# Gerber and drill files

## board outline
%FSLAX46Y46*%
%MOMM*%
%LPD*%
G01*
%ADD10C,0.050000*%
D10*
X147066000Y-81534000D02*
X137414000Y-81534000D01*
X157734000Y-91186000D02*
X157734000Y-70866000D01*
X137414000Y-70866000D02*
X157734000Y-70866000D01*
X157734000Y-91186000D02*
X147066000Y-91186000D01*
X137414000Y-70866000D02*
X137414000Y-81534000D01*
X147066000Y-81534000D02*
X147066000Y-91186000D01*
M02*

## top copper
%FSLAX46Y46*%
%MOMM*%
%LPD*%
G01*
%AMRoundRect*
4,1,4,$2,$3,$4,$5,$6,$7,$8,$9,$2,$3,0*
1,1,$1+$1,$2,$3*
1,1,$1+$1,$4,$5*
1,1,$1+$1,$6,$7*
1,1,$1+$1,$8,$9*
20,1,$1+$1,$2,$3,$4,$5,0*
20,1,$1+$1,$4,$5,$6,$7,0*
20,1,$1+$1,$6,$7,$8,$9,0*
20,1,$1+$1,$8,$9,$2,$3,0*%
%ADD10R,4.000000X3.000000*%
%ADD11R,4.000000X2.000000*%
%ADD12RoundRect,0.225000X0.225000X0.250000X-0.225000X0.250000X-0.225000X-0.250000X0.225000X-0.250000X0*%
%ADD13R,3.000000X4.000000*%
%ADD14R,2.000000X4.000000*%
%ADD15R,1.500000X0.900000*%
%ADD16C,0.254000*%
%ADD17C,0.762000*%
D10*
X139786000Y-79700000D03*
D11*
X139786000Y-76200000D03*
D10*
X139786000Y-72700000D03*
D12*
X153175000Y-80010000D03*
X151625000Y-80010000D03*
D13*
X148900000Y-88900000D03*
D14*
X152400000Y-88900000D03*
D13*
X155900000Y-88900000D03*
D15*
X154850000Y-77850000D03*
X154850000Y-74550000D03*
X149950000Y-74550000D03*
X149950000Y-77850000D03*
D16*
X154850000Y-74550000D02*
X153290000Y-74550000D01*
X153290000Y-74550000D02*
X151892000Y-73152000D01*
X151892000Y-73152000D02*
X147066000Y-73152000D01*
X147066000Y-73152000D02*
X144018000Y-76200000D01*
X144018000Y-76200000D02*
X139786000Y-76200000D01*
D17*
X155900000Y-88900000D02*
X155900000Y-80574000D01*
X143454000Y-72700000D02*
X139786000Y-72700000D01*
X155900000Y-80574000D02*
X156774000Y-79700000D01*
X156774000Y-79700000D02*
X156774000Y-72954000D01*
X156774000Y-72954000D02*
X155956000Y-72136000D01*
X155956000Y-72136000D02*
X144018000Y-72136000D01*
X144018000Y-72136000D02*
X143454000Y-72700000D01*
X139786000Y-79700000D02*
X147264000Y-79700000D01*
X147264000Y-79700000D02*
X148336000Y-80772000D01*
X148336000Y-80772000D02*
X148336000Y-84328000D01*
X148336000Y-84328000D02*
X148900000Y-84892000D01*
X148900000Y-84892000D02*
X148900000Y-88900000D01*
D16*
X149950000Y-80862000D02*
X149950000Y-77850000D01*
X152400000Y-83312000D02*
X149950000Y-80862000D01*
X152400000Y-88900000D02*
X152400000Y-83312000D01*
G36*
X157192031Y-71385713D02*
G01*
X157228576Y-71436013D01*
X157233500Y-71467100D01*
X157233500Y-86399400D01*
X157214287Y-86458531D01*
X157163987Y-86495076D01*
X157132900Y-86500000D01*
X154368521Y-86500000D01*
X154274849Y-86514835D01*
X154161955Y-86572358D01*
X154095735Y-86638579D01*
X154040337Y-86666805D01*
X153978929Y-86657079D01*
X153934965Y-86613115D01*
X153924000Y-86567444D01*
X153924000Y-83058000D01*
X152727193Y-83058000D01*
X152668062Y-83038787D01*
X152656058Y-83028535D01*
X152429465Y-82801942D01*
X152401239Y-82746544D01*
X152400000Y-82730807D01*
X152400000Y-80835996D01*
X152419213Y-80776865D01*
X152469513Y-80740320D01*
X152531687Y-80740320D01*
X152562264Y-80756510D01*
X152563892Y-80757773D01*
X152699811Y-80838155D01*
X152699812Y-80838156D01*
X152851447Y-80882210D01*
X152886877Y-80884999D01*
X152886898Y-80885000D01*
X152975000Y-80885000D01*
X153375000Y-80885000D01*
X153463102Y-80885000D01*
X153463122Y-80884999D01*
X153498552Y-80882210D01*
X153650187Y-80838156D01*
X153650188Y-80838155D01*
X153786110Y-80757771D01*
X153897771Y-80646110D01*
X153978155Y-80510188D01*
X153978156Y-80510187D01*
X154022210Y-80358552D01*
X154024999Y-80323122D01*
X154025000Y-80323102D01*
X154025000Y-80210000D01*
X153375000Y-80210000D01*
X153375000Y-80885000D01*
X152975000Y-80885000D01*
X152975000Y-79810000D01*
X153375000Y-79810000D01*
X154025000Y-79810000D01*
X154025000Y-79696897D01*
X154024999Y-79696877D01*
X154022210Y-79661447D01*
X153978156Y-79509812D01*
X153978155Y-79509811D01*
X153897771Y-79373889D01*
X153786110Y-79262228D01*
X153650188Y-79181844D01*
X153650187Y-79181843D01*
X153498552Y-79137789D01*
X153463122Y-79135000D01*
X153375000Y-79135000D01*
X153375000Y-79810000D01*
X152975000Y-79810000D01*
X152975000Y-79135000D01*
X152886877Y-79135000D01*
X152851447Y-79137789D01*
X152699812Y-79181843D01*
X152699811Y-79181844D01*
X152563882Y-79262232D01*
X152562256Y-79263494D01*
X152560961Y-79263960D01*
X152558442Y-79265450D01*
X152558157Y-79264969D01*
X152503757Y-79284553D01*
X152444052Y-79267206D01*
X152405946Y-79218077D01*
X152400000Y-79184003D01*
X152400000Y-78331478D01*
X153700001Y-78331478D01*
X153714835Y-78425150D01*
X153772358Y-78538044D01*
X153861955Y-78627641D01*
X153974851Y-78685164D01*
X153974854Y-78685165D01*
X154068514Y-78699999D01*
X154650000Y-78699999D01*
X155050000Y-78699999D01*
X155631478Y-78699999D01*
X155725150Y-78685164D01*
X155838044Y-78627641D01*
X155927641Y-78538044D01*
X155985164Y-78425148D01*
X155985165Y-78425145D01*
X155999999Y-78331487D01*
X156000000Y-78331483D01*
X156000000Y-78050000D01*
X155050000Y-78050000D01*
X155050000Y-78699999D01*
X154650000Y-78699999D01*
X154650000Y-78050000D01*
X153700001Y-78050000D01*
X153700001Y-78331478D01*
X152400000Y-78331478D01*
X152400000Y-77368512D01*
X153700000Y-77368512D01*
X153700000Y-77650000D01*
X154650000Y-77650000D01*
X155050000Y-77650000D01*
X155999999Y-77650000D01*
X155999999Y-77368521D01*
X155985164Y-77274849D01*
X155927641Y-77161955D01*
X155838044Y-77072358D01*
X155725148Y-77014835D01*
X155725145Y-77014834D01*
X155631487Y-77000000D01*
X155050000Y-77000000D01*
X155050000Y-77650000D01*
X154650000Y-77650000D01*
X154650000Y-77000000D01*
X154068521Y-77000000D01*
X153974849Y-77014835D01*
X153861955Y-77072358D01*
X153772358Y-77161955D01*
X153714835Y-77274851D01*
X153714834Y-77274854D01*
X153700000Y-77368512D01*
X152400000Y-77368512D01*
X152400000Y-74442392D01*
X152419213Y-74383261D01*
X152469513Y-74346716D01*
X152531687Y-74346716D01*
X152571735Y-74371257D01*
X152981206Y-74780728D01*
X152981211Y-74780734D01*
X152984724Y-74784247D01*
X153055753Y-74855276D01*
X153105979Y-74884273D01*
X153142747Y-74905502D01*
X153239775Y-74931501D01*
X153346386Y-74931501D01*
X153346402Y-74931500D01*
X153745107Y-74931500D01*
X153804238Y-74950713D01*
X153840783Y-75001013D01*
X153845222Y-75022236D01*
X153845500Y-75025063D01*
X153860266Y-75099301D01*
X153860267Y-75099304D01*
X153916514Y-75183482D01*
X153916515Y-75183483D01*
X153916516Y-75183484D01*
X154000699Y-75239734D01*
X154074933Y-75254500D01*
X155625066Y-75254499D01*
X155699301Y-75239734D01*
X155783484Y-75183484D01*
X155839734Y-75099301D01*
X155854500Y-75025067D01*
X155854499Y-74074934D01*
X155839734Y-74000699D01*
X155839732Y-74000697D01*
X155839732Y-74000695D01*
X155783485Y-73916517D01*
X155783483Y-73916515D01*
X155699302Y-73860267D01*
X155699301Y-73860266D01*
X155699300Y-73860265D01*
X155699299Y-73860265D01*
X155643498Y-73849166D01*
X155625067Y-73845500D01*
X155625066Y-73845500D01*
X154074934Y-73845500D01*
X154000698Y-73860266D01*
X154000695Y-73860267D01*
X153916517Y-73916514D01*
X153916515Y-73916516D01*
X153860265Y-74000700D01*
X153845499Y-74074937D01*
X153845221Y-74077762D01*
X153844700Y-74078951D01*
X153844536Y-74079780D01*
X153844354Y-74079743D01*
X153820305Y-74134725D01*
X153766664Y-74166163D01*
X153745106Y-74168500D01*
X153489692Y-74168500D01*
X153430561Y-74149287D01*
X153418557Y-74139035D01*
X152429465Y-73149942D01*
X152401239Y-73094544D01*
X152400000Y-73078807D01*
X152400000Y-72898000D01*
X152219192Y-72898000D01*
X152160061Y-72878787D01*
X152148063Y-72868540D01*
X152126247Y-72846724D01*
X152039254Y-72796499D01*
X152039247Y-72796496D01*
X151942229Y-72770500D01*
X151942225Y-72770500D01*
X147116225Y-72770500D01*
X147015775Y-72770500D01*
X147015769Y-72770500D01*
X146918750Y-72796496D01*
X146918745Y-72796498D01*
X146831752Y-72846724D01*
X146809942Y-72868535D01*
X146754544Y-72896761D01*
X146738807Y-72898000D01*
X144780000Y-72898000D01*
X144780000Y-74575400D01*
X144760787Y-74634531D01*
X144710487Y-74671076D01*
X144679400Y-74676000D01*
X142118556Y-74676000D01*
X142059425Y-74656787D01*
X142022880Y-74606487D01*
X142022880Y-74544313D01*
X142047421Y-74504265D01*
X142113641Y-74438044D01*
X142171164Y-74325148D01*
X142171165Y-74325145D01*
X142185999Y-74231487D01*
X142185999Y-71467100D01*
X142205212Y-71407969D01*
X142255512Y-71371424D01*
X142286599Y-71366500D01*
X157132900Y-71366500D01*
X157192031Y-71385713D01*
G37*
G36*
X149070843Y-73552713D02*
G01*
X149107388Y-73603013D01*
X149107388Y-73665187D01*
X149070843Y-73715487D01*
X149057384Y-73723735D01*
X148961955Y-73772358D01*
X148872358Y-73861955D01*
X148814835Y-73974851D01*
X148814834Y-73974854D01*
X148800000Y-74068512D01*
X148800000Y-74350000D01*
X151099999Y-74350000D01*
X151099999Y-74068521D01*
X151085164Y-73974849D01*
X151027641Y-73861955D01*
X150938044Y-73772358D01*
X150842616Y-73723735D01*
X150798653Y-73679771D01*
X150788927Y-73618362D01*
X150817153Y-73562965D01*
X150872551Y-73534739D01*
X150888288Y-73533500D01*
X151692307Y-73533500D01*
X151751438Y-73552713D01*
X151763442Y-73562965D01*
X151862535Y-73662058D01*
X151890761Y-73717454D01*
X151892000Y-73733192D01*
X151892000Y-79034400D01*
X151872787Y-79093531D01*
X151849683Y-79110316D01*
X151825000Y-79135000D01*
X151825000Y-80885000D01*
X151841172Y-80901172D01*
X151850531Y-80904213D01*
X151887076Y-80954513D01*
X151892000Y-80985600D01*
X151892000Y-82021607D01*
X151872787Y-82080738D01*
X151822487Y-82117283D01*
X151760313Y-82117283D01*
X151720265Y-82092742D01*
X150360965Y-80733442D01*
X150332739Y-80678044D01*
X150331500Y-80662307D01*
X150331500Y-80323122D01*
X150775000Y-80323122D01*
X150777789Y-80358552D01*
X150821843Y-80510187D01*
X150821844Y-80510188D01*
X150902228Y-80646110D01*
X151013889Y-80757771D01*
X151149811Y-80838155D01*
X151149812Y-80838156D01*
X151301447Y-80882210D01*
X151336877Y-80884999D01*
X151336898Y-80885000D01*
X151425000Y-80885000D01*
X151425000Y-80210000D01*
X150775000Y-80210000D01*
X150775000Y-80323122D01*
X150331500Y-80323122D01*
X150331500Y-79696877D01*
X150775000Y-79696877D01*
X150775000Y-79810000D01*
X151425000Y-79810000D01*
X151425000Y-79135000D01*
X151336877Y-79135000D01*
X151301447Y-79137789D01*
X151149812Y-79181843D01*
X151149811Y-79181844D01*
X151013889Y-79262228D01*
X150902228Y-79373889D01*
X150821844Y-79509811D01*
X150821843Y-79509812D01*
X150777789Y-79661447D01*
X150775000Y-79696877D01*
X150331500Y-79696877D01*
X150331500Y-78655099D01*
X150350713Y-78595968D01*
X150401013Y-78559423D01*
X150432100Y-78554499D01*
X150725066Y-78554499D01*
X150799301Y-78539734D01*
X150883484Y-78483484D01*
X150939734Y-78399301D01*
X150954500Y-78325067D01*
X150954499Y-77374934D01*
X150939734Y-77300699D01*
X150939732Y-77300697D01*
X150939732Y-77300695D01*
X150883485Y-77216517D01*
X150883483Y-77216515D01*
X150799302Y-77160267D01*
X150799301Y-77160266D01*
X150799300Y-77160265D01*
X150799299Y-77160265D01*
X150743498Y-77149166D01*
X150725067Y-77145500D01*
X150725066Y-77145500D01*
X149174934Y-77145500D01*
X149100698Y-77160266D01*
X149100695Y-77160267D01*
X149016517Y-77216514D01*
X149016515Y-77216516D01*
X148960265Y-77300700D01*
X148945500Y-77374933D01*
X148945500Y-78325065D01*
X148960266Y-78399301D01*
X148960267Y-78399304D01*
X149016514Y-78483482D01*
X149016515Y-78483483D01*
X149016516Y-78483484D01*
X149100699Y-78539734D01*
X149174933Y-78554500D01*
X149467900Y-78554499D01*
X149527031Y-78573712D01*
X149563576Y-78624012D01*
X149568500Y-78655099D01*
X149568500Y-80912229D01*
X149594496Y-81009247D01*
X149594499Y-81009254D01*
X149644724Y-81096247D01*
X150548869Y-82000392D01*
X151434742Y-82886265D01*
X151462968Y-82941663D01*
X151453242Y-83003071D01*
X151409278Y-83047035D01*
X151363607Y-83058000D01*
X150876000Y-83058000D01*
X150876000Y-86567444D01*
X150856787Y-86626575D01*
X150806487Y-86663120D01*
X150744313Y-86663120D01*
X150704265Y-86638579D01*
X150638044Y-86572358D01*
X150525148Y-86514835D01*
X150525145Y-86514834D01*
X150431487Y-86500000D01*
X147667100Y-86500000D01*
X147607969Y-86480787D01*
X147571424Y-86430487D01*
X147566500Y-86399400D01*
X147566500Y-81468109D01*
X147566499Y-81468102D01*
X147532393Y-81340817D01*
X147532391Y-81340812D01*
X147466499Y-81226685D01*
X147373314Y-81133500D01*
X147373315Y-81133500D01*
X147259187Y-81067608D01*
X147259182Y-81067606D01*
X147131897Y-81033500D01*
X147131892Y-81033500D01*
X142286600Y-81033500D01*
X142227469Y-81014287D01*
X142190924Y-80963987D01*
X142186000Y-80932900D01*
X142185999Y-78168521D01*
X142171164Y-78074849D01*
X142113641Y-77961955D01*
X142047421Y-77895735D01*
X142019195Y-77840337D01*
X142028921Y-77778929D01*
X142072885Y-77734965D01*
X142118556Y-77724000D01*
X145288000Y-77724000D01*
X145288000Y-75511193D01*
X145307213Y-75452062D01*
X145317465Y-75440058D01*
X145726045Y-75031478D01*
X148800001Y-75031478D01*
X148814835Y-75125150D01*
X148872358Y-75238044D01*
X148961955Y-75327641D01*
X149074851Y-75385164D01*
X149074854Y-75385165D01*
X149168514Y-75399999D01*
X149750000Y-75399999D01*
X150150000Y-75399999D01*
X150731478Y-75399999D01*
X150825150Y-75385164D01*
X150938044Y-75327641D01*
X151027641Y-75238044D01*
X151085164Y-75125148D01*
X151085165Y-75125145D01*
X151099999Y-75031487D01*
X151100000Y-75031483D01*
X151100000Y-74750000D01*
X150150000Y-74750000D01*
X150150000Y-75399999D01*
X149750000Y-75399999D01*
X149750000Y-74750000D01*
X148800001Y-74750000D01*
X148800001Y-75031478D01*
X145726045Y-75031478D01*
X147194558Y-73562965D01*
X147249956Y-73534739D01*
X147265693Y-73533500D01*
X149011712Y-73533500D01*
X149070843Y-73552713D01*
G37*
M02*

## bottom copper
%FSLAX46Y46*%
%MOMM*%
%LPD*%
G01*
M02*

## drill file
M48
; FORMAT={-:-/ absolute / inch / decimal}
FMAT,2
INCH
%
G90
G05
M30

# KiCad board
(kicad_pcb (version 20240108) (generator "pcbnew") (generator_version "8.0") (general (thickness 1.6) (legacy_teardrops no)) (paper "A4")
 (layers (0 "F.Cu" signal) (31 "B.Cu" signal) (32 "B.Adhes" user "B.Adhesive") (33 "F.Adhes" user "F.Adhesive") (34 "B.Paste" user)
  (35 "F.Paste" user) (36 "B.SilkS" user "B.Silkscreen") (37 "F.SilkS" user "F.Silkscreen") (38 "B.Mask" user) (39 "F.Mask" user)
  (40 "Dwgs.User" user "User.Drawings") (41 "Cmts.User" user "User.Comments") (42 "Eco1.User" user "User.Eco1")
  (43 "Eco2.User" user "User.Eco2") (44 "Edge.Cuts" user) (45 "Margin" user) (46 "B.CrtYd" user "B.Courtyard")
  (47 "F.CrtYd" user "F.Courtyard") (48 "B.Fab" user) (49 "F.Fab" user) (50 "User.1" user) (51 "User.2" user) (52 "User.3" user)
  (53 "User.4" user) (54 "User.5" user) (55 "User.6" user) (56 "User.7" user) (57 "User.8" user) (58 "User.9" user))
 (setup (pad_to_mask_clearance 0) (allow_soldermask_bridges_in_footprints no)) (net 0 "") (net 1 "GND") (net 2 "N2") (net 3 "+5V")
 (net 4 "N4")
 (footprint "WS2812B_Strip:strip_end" (layer "F.Cu") (at 139.786 76.2 180)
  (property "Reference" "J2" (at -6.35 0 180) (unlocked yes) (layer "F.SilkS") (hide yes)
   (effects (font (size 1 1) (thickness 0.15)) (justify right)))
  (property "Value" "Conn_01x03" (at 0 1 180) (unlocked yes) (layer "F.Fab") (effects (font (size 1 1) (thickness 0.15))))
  (pad "1" smd rect (at 0 -3.5 180) (size 4 3) (layers "F.Cu" "F.Paste" "F.Mask") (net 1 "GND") (thermal_bridge_angle 45))
  (pad "2" smd rect (at 0 0 180) (size 4 2) (layers "F.Cu" "F.Paste" "F.Mask") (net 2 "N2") (thermal_bridge_angle 45))
  (pad "3" smd rect (at 0 3.5 180) (size 4 3) (layers "F.Cu" "F.Paste" "F.Mask") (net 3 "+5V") (thermal_bridge_angle 45)))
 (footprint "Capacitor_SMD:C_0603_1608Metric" (layer "F.Cu") (at 152.4 80.01 180)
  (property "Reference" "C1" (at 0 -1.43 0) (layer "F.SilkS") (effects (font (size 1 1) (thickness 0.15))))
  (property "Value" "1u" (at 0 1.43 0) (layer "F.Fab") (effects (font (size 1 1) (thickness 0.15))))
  (pad "1" smd roundrect (at -0.775 0 180) (size 0.9 0.95) (layers "F.Cu" "F.Paste" "F.Mask") (roundrect_rratio 0.25) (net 3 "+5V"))
  (pad "2" smd roundrect (at 0.775 0 180) (size 0.9 0.95) (layers "F.Cu" "F.Paste" "F.Mask") (roundrect_rratio 0.25) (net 1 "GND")))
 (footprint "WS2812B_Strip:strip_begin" (layer "F.Cu") (at 152.4 88.9 90)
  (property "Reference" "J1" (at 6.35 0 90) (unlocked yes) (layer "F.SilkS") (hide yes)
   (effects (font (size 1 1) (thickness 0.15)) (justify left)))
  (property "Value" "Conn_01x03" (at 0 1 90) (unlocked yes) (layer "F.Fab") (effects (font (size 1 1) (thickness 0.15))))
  (pad "1" smd rect (at 0 -3.5 90) (size 4 3) (layers "F.Cu" "F.Paste" "F.Mask") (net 1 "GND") (thermal_bridge_angle 45))
  (pad "2" smd rect (at 0 0 90) (size 4 2) (layers "F.Cu" "F.Paste" "F.Mask") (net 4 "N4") (thermal_bridge_angle 45))
  (pad "3" smd rect (at 0 3.5 90) (size 4 3) (layers "F.Cu" "F.Paste" "F.Mask") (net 3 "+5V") (thermal_bridge_angle 45)))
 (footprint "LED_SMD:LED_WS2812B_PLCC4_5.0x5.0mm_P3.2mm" (layer "F.Cu") (at 152.4 76.2 180)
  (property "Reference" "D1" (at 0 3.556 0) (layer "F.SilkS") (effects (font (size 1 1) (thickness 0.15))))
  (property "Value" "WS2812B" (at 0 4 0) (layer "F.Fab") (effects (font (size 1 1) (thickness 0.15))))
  (pad "1" smd rect (at -2.45 -1.65 180) (size 1.5 0.9) (layers "F.Cu" "F.Paste" "F.Mask") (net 3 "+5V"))
  (pad "2" smd rect (at -2.45 1.65 180) (size 1.5 0.9) (layers "F.Cu" "F.Paste" "F.Mask") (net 2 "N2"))
  (pad "3" smd rect (at 2.45 1.65 180) (size 1.5 0.9) (layers "F.Cu" "F.Paste" "F.Mask") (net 1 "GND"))
  (pad "4" smd rect (at 2.45 -1.65 180) (size 1.5 0.9) (layers "F.Cu" "F.Paste" "F.Mask") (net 4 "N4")))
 (gr_line (start 147.066 81.534) (end 137.414 81.534) (stroke (width 0.05) (type default)) (layer "Edge.Cuts"))
 (gr_line (start 157.734 91.186) (end 157.734 70.866) (stroke (width 0.05) (type default)) (layer "Edge.Cuts"))
 (gr_line (start 137.414 70.866) (end 157.734 70.866) (stroke (width 0.05) (type default)) (layer "Edge.Cuts"))
 (gr_line (start 157.734 91.186) (end 147.066 91.186) (stroke (width 0.05) (type default)) (layer "Edge.Cuts"))
 (gr_line (start 137.414 70.866) (end 137.414 81.534) (stroke (width 0.05) (type default)) (layer "Edge.Cuts"))
 (gr_line (start 147.066 81.534) (end 147.066 91.186) (stroke (width 0.05) (type default)) (layer "Edge.Cuts"))
 (segment (start 149.95 80.862) (end 149.95 77.85) (width 0.254) (layer "F.Cu") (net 4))
 (segment (start 152.4 83.312) (end 149.95 80.862) (width 0.254) (layer "F.Cu") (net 4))
 (segment (start 152.4 88.9) (end 152.4 83.312) (width 0.254) (layer "F.Cu") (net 4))
 (segment (start 144.018 76.2) (end 139.786 76.2) (width 0.254) (layer "F.Cu") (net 2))
 (segment (start 154.85 74.55) (end 153.29 74.55) (width 0.254) (layer "F.Cu") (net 2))
 (segment (start 151.892 73.152) (end 147.066 73.152) (width 0.254) (layer "F.Cu") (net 2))
 (segment (start 153.29 74.55) (end 151.892 73.152) (width 0.254) (layer "F.Cu") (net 2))
 (segment (start 147.066 73.152) (end 144.018 76.2) (width 0.254) (layer "F.Cu") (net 2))
 (segment (start 148.336 80.772) (end 148.336 84.328) (width 0.762) (layer "F.Cu") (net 1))
 (segment (start 139.786 79.7) (end 147.264 79.7) (width 0.762) (layer "F.Cu") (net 1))
 (segment (start 147.264 79.7) (end 148.336 80.772) (width 0.762) (layer "F.Cu") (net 1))
 (segment (start 148.9 84.892) (end 148.9 88.9) (width 0.762) (layer "F.Cu") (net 1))
 (segment (start 148.336 84.328) (end 148.9 84.892) (width 0.762) (layer "F.Cu") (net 1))
 (segment (start 156.774 72.954) (end 155.956 72.136) (width 0.762) (layer "F.Cu") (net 3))
 (segment (start 155.9 80.574) (end 156.774 79.7) (width 0.762) (layer "F.Cu") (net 3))
 (segment (start 155.956 72.136) (end 144.018 72.136) (width 0.762) (layer "F.Cu") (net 3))
 (segment (start 143.454 72.7) (end 139.786 72.7) (width 0.762) (layer "F.Cu") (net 3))
 (segment (start 144.018 72.136) (end 143.454 72.7) (width 0.762) (layer "F.Cu") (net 3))
 (segment (start 156.774 79.7) (end 156.774 72.954) (width 0.762) (layer "F.Cu") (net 3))
 (segment (start 155.9 88.9) (end 155.9 80.574) (width 0.762) (layer "F.Cu") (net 3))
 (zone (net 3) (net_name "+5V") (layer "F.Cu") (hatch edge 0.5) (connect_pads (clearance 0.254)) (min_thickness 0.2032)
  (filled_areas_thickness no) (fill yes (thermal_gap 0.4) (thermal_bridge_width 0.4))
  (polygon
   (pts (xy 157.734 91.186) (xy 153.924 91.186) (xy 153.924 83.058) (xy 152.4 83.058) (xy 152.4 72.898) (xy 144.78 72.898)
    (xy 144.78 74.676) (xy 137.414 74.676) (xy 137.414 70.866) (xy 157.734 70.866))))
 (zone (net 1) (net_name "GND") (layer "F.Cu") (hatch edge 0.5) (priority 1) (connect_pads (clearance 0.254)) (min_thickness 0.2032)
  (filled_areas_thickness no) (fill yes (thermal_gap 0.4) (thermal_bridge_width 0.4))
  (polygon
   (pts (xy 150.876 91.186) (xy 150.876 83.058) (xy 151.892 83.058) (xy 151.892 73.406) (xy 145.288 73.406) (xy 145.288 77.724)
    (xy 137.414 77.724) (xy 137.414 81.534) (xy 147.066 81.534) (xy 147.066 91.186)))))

